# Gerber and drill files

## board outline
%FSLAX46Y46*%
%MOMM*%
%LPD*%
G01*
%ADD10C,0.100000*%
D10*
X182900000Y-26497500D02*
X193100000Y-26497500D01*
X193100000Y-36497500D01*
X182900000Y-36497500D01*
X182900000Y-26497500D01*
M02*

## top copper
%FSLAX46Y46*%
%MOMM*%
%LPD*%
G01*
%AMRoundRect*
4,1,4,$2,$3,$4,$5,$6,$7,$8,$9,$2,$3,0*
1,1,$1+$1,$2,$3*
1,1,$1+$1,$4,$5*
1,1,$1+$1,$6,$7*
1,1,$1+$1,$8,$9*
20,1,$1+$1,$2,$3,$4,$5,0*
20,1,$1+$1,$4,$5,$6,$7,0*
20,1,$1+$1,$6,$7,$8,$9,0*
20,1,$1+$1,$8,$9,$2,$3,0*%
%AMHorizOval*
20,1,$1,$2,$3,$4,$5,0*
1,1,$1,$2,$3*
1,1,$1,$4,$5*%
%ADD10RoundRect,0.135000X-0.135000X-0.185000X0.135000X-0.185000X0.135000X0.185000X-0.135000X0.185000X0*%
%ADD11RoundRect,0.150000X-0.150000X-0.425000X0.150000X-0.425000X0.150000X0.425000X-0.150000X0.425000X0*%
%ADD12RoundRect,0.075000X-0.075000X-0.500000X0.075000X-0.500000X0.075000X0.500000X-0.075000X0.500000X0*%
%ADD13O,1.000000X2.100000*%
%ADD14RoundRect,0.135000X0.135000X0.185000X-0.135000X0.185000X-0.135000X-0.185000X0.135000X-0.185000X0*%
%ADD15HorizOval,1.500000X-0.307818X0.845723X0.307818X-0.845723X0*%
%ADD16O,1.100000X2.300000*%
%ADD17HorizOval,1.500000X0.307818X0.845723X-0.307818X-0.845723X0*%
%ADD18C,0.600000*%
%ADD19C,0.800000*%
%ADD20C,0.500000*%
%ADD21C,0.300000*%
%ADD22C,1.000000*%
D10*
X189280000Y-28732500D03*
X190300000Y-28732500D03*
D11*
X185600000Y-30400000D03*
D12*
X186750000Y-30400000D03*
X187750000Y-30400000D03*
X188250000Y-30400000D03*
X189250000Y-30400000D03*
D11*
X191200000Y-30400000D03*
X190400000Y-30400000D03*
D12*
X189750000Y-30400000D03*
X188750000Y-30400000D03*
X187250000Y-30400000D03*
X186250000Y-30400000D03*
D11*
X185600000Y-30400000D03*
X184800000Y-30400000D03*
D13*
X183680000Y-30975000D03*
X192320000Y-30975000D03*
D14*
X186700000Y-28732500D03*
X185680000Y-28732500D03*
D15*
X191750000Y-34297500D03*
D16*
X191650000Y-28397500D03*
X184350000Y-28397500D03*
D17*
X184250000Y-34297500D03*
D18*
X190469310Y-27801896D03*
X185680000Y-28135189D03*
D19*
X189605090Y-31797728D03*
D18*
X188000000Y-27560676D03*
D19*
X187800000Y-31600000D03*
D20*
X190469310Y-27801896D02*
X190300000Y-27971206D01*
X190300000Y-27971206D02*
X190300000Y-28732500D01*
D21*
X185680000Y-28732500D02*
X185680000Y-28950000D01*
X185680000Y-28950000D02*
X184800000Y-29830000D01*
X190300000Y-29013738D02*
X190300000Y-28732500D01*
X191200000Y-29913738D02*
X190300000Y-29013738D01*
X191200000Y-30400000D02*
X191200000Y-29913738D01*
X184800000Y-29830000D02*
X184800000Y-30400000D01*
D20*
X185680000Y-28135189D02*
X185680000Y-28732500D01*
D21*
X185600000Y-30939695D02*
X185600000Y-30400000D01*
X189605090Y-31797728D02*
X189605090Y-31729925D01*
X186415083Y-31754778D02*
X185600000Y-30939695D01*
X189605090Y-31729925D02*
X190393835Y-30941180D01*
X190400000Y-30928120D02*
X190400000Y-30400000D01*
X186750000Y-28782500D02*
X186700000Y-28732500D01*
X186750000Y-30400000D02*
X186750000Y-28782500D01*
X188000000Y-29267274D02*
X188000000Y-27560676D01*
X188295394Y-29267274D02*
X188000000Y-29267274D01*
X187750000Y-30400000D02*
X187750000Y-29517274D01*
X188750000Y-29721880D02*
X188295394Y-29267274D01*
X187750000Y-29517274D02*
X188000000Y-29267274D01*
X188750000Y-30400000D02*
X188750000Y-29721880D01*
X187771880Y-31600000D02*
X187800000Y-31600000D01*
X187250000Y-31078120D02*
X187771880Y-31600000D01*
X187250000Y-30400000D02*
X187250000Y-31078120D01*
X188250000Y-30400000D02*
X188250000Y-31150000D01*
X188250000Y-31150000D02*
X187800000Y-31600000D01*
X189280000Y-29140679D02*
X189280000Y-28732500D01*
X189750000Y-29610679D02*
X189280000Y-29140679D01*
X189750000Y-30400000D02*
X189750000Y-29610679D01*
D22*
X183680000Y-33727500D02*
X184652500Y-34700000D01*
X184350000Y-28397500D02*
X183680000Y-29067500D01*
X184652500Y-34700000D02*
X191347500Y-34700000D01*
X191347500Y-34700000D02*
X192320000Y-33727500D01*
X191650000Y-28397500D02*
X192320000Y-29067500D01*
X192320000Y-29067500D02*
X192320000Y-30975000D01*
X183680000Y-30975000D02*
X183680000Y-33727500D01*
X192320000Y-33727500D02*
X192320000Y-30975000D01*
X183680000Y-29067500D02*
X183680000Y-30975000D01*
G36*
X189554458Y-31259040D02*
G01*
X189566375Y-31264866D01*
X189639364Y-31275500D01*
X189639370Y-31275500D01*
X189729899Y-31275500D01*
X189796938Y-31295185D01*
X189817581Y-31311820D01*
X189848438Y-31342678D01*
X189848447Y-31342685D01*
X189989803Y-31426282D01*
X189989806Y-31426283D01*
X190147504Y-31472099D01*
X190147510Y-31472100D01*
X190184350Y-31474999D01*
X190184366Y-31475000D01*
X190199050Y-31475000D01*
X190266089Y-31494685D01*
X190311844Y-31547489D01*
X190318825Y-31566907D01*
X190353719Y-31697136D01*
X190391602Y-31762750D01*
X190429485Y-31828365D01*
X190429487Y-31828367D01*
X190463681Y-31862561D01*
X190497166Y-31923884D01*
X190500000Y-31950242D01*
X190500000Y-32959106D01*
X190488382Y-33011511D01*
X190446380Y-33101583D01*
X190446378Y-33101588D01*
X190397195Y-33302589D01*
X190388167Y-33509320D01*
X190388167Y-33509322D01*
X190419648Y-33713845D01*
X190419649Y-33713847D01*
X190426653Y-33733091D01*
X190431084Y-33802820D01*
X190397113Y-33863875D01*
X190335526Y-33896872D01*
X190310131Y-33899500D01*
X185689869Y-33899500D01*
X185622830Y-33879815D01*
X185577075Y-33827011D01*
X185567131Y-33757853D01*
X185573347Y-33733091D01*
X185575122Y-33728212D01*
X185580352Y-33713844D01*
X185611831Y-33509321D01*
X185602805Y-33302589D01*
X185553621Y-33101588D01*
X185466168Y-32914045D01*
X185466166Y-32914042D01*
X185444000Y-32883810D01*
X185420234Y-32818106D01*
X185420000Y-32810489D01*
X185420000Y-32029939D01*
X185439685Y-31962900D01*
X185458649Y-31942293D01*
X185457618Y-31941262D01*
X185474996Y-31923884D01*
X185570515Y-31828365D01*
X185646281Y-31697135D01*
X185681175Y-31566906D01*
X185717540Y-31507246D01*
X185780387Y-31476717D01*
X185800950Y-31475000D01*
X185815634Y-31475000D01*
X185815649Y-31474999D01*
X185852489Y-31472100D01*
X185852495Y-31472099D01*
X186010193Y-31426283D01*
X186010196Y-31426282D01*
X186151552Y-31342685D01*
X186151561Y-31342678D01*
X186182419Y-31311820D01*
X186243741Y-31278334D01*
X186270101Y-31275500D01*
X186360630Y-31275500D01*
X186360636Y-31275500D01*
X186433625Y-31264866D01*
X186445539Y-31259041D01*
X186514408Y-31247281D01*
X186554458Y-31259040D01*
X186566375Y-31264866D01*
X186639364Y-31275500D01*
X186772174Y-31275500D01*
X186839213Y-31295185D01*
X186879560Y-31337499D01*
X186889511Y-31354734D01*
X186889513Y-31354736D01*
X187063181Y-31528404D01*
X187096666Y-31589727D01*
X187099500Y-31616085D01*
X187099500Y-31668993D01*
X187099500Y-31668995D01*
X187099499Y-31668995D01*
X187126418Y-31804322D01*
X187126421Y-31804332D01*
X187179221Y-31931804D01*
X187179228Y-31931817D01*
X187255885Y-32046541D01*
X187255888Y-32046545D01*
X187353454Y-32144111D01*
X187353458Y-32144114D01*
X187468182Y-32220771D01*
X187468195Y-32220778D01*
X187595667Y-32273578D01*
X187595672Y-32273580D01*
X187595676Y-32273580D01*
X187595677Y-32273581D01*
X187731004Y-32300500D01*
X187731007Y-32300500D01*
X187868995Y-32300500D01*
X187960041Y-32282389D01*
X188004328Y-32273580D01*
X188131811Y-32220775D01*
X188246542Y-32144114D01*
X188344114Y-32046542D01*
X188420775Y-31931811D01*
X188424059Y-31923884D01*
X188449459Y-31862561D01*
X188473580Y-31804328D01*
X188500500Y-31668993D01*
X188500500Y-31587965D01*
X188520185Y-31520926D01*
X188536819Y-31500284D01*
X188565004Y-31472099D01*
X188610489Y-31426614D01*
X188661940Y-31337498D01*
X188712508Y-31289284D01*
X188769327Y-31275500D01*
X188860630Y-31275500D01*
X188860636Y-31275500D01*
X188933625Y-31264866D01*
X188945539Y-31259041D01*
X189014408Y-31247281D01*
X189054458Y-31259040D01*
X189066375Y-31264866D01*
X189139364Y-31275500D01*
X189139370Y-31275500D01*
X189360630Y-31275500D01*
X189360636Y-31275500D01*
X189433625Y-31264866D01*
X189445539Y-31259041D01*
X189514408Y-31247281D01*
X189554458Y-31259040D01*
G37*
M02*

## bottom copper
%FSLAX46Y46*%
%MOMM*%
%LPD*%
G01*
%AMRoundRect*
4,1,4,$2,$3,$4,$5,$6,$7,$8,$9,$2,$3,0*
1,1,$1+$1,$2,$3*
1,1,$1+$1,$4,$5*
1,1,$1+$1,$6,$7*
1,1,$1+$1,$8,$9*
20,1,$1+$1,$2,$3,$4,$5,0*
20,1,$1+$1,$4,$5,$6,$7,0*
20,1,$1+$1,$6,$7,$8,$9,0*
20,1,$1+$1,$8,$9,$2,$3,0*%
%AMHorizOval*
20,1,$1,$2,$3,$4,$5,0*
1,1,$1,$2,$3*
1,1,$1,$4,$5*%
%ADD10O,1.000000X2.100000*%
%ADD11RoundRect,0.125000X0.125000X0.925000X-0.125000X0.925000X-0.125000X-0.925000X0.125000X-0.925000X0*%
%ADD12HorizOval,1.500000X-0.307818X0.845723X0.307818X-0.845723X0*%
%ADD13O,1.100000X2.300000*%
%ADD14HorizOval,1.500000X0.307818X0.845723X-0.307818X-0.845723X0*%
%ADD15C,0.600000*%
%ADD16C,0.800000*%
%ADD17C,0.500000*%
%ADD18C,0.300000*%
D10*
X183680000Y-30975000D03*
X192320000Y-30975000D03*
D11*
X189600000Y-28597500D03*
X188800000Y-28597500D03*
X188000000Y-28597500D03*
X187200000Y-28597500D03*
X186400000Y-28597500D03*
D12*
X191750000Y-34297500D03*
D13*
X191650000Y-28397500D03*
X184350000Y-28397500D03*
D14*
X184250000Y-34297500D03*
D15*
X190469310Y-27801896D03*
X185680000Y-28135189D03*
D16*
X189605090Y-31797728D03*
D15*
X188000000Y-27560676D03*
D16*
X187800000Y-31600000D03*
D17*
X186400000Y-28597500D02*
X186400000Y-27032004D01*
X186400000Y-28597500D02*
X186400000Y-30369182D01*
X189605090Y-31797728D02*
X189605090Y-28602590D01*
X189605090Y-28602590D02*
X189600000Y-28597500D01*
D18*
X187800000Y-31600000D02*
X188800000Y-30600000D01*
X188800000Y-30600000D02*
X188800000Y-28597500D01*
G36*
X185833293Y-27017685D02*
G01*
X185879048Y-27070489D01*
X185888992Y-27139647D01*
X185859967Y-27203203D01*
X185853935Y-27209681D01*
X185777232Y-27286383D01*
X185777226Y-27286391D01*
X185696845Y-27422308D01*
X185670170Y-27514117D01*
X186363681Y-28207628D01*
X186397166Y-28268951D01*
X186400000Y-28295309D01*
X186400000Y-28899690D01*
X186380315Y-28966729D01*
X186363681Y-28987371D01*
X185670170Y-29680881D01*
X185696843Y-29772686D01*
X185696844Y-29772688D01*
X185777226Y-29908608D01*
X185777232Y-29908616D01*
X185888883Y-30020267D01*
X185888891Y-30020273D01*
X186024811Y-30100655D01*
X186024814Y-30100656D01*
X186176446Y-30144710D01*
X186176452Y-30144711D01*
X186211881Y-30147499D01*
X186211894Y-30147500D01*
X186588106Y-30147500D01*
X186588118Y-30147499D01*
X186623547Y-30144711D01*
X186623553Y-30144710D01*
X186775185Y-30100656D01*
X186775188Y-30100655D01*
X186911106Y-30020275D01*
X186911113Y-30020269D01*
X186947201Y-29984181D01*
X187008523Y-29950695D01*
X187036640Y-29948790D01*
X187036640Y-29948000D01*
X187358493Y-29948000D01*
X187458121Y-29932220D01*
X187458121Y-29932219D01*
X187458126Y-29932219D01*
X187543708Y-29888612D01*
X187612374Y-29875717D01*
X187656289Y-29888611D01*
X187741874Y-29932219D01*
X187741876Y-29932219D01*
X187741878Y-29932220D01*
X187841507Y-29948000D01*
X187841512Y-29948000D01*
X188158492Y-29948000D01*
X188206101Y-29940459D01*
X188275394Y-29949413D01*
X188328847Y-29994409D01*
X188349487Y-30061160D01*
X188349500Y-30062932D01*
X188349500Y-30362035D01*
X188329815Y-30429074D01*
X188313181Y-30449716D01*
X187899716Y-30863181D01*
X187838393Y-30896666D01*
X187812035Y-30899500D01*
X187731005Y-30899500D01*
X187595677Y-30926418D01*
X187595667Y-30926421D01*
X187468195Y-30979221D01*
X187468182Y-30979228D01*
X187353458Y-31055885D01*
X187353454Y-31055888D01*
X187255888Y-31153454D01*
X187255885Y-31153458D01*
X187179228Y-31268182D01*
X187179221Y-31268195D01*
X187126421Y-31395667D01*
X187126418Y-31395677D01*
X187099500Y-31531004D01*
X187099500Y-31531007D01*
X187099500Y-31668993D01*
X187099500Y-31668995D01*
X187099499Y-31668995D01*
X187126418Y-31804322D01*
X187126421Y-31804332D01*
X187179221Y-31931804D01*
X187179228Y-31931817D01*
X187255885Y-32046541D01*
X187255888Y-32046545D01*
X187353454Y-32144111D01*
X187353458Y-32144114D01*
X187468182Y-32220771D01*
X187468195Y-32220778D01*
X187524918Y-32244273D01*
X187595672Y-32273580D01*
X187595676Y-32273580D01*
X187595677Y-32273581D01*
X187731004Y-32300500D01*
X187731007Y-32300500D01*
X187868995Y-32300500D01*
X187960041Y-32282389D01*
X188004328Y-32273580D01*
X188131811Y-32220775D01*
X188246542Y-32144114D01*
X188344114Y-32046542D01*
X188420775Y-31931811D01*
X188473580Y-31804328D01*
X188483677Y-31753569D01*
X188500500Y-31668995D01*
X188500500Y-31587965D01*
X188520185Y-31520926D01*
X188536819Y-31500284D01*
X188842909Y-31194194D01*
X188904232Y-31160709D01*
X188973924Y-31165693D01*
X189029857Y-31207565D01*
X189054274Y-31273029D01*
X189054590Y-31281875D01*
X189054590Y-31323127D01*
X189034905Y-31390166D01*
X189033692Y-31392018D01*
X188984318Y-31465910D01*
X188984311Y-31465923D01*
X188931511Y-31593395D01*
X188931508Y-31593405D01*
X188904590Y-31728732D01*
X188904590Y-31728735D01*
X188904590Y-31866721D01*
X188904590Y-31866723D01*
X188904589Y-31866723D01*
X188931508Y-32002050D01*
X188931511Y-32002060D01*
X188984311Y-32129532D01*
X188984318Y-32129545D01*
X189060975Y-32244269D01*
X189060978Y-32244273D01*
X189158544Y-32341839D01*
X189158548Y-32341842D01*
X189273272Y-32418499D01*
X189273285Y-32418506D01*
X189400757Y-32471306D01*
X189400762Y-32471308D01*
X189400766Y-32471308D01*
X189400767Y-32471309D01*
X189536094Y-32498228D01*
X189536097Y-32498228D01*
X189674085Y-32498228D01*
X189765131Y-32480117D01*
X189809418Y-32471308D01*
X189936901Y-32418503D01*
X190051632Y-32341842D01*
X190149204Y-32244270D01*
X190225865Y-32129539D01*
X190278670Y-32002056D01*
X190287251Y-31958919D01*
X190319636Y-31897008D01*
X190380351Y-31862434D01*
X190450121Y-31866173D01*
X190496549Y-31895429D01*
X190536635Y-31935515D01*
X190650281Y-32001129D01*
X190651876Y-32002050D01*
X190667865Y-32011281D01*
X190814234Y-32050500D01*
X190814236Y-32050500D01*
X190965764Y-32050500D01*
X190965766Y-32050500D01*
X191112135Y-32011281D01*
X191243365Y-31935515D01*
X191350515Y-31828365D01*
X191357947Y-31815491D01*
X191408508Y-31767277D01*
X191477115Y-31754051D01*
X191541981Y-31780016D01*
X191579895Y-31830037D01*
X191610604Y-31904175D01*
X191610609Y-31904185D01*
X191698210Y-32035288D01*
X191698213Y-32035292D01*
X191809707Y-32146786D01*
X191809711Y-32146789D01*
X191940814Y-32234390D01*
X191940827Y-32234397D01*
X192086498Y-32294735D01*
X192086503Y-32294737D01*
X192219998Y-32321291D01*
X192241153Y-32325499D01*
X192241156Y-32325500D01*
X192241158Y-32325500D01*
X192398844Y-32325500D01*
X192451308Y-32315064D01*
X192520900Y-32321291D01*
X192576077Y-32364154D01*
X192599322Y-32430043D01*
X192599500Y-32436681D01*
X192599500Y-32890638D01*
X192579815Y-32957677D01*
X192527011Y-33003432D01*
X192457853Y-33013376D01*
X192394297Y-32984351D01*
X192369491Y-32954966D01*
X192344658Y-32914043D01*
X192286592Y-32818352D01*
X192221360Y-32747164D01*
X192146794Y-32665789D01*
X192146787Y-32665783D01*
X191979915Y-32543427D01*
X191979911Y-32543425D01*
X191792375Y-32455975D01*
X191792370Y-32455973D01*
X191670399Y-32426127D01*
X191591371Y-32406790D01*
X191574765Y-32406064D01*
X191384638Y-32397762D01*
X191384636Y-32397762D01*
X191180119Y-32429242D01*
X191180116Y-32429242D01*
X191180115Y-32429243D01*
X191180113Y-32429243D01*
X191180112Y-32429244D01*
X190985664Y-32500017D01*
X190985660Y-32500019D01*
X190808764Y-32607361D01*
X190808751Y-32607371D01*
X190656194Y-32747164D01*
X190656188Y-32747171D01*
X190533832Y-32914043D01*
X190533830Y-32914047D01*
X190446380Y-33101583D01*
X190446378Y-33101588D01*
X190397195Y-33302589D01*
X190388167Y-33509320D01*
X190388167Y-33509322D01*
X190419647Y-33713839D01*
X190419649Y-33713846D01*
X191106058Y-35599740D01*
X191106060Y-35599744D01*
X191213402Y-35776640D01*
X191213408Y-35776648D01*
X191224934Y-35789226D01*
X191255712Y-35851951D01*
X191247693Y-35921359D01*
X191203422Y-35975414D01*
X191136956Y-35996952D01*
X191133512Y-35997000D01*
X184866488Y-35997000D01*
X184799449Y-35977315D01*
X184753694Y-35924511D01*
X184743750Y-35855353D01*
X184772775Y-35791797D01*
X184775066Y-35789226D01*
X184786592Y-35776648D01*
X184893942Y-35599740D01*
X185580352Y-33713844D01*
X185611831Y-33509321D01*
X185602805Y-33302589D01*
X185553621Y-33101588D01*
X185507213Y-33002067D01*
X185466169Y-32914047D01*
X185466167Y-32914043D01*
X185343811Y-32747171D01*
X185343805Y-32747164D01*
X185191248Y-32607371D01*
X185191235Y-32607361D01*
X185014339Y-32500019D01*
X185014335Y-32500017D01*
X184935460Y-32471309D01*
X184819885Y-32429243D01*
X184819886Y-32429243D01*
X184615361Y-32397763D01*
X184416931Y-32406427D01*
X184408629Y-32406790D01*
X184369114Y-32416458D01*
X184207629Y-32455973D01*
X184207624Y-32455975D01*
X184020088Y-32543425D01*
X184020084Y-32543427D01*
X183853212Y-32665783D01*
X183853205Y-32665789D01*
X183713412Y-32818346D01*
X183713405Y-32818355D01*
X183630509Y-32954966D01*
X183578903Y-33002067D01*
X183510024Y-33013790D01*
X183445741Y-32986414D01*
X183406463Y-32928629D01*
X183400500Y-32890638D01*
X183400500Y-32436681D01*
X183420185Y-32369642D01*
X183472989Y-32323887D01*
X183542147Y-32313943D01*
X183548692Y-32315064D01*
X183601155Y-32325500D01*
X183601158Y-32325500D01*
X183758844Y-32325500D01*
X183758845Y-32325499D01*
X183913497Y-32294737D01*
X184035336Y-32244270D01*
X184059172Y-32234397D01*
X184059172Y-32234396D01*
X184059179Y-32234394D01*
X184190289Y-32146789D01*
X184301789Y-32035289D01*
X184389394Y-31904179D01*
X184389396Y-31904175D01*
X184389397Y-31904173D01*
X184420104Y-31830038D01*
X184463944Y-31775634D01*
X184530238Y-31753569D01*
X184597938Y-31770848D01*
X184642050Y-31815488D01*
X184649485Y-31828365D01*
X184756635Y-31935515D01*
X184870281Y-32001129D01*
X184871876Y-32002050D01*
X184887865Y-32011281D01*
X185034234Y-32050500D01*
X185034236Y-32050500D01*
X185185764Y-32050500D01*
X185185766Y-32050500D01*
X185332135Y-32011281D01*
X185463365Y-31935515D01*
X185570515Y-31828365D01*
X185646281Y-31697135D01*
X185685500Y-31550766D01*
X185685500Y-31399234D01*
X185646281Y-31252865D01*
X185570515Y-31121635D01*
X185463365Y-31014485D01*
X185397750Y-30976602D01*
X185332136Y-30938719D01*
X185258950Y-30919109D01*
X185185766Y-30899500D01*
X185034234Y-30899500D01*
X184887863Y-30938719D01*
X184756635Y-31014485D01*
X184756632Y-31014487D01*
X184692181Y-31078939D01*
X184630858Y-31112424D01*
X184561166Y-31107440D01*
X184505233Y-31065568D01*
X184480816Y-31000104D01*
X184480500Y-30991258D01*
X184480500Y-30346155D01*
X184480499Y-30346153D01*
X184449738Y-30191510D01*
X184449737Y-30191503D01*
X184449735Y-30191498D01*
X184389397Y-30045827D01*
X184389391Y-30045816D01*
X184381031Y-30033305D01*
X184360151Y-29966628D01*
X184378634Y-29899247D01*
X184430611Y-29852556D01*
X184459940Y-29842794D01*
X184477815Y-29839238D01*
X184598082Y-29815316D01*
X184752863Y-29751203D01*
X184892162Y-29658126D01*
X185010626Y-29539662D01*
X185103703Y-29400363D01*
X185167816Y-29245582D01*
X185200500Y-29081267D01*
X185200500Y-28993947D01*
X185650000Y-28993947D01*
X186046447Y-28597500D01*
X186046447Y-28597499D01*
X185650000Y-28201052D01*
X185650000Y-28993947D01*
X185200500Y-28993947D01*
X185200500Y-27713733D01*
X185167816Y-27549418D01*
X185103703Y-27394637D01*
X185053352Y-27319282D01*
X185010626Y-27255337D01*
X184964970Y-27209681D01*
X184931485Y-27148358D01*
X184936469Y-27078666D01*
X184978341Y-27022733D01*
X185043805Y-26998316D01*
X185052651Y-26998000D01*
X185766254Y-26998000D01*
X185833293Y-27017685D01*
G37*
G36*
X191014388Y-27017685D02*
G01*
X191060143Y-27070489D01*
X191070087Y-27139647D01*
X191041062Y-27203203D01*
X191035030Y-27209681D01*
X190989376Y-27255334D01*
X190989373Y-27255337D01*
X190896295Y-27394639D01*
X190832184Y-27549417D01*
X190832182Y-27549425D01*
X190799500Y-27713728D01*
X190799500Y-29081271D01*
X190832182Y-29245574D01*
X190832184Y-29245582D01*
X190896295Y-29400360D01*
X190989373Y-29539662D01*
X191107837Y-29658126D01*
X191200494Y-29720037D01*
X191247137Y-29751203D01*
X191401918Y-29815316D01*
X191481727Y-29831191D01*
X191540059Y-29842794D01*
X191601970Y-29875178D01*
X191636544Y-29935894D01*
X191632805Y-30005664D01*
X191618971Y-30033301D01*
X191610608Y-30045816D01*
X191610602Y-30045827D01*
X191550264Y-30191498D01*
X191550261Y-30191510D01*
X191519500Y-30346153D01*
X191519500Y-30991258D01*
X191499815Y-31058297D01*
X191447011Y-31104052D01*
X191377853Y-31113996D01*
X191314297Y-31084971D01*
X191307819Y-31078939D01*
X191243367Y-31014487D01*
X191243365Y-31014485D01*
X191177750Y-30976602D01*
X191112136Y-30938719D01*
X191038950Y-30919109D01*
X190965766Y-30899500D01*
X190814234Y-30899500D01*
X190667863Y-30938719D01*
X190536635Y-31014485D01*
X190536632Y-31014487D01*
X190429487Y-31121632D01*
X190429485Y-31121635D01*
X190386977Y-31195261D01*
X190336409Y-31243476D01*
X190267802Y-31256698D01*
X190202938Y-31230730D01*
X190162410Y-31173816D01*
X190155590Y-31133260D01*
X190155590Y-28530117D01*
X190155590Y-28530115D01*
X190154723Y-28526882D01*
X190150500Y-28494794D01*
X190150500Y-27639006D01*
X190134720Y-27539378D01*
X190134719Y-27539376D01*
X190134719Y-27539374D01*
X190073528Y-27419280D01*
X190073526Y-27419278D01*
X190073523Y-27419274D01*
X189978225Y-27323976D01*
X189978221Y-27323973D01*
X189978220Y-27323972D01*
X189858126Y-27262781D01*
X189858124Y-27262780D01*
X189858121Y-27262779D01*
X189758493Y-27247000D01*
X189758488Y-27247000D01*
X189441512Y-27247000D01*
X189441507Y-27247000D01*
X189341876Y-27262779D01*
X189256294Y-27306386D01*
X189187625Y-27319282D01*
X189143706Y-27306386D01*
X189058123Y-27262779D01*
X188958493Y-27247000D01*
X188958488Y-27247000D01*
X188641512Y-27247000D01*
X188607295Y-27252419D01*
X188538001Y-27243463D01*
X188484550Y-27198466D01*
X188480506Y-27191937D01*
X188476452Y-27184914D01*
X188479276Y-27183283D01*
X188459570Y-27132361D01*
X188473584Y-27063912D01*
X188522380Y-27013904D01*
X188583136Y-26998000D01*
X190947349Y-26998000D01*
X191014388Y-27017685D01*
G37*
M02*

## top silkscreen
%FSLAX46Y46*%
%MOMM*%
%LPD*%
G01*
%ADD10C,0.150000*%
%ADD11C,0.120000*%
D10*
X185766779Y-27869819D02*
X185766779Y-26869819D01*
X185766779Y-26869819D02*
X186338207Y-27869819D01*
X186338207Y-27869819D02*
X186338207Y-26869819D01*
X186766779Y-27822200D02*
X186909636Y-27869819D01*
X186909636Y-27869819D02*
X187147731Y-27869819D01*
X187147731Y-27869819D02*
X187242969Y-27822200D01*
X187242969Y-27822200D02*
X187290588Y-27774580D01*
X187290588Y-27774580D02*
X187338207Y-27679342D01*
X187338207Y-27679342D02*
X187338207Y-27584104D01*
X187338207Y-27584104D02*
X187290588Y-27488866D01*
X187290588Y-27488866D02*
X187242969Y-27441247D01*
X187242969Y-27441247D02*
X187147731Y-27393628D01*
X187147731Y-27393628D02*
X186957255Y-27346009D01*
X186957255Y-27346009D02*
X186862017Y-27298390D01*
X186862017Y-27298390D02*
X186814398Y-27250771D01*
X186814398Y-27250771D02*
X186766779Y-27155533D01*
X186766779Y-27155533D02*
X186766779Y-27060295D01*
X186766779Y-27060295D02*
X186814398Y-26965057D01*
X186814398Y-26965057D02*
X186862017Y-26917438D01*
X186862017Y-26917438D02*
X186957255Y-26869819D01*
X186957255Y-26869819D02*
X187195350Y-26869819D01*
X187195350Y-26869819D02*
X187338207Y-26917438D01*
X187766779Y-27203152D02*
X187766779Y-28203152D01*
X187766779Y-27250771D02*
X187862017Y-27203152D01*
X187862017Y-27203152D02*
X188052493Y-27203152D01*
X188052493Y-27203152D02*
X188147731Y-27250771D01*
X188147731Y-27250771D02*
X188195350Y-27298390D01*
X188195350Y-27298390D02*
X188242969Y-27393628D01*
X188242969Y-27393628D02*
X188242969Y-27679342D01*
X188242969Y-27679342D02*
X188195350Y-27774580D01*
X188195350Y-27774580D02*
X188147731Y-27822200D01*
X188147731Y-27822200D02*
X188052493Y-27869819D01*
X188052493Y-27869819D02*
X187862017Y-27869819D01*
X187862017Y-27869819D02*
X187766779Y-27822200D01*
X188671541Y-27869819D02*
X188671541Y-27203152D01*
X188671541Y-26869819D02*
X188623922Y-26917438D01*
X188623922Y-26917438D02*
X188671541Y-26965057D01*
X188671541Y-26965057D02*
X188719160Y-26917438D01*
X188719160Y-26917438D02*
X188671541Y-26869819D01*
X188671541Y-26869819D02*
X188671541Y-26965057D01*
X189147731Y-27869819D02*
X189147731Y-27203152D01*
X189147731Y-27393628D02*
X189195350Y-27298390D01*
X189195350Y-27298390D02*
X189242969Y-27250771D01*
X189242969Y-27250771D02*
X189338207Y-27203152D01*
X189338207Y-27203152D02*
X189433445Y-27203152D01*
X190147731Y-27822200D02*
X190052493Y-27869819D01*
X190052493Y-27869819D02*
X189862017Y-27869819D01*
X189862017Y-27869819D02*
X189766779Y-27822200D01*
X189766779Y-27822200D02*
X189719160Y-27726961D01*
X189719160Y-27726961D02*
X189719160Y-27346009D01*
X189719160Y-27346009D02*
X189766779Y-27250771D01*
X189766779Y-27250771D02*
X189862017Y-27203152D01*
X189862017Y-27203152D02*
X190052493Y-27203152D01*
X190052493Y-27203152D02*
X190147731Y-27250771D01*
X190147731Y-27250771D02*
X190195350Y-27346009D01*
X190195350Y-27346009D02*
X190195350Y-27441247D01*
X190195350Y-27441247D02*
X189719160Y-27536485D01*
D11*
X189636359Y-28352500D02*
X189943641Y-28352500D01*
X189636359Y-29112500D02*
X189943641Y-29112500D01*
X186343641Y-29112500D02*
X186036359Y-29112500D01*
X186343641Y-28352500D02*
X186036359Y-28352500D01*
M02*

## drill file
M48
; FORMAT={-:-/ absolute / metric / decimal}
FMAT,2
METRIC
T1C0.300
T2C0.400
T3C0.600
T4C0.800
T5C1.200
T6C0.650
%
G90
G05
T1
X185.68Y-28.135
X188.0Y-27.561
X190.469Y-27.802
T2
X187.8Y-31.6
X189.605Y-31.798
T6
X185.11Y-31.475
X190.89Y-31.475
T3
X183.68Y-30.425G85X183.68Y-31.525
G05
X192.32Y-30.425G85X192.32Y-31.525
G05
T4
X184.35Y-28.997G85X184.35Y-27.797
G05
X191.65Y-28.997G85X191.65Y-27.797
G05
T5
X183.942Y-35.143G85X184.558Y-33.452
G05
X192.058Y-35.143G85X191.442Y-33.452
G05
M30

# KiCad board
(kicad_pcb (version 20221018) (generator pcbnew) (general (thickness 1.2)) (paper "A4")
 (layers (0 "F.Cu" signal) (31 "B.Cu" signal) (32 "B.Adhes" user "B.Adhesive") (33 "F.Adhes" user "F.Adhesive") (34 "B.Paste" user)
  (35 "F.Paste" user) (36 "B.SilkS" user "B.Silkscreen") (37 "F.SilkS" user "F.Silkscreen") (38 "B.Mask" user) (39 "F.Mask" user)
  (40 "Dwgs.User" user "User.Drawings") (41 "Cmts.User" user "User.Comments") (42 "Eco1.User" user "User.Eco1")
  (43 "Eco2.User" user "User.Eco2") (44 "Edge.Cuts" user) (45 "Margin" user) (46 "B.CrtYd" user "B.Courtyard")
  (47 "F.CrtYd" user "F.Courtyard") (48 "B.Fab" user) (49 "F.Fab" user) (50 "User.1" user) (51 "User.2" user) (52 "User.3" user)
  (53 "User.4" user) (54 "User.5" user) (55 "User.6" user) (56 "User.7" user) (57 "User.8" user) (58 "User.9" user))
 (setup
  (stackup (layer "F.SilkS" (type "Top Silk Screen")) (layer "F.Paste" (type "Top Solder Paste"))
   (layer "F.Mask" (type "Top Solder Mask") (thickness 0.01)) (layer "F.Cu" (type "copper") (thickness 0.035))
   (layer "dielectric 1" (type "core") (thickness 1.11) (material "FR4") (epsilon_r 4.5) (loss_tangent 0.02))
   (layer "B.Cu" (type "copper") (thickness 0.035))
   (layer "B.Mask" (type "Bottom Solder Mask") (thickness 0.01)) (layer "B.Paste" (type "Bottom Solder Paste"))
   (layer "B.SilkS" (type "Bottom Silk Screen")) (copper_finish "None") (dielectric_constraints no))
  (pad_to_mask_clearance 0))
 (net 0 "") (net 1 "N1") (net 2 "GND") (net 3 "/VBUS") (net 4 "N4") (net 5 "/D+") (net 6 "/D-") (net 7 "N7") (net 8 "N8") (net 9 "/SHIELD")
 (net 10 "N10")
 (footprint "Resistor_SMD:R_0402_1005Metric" (layer "F.Cu") (at 189.79 28.7325)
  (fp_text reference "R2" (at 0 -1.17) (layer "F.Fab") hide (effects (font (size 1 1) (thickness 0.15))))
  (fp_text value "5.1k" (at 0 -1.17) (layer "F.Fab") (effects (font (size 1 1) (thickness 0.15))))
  (fp_line (start -0.153641 -0.38) (end 0.153641 -0.38) (stroke (width 0.12) (type solid)) (layer "F.SilkS"))
  (fp_line (start -0.153641 0.38) (end 0.153641 0.38) (stroke (width 0.12) (type solid)) (layer "F.SilkS"))
  (pad "1" smd roundrect (at -0.51 0) (size 0.54 0.64) (layers "F.Cu" "F.Paste" "F.Mask") (roundrect_rratio 0.25) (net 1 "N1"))
  (pad "2" smd roundrect (at 0.51 0) (size 0.54 0.64) (layers "F.Cu" "F.Paste" "F.Mask") (roundrect_rratio 0.25) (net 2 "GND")))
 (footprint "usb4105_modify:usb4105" (layer "F.Cu") (at 187.98 39.92)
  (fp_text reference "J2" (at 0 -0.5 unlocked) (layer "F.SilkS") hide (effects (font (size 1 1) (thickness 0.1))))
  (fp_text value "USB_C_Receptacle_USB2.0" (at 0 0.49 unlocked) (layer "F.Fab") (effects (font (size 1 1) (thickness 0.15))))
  (pad "" np_thru_hole circle (at -2.87 -8.445) (size 0.65 0.65) (drill 0.65) (layers "F&B.Cu" "*.Mask"))
  (pad "" np_thru_hole circle (at 2.91 -8.445) (size 0.65 0.65) (drill 0.65) (layers "F&B.Cu" "*.Mask"))
  (pad "A4" smd roundrect (at -2.38 -9.52) (size 0.6 1.15) (layers "F.Cu" "F.Paste" "F.Mask") (roundrect_rratio 0.25) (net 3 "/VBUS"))
  (pad "A5" smd roundrect (at -1.23 -9.52) (size 0.3 1.15) (layers "F.Cu" "F.Paste" "F.Mask") (roundrect_rratio 0.25) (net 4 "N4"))
  (pad "A6" smd roundrect (at -0.23 -9.52) (size 0.3 1.15) (layers "F.Cu" "F.Paste" "F.Mask") (roundrect_rratio 0.25) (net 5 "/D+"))
  (pad "A7" smd roundrect (at 0.27 -9.52) (size 0.3 1.15) (layers "F.Cu" "F.Paste" "F.Mask") (roundrect_rratio 0.25) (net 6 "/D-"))
  (pad "A8" smd roundrect (at 1.27 -9.52) (size 0.3 1.15) (layers "F.Cu" "F.Paste" "F.Mask") (roundrect_rratio 0.25) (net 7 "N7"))
  (pad "A12" smd roundrect (at 3.22 -9.52) (size 0.6 1.15) (layers "F.Cu" "F.Paste" "F.Mask") (roundrect_rratio 0.25) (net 2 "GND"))
  (pad "B4" smd roundrect (at 2.42 -9.52) (size 0.6 1.15) (layers "F.Cu" "F.Paste" "F.Mask") (roundrect_rratio 0.25) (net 3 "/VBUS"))
  (pad "B5" smd roundrect (at 1.77 -9.52) (size 0.3 1.15) (layers "F.Cu" "F.Paste" "F.Mask") (roundrect_rratio 0.25) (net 1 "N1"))
  (pad "B6" smd roundrect (at 0.77 -9.52) (size 0.3 1.15) (layers "F.Cu" "F.Paste" "F.Mask") (roundrect_rratio 0.25) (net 5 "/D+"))
  (pad "B7" smd roundrect (at -0.73 -9.52) (size 0.3 1.15) (layers "F.Cu" "F.Paste" "F.Mask") (roundrect_rratio 0.25) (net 6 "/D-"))
  (pad "B8" smd roundrect (at -1.73 -9.52) (size 0.3 1.15) (layers "F.Cu" "F.Paste" "F.Mask") (roundrect_rratio 0.25) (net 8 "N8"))
  (pad "B9" smd roundrect (at -2.38 -9.52) (size 0.6 1.15) (layers "F.Cu" "F.Paste" "F.Mask") (roundrect_rratio 0.25) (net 3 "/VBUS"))
  (pad "B12" smd roundrect (at -3.18 -9.52) (size 0.6 1.15) (layers "F.Cu" "F.Paste" "F.Mask") (roundrect_rratio 0.25) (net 2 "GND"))
  (pad "S1" thru_hole oval (at -4.3 -8.945) (size 1 2.1) (drill oval 0.6 1.7) (layers "*.Cu" "*.Mask" "F.Paste") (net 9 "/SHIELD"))
  (pad "S1" thru_hole oval (at 4.34 -8.945) (size 1 2.1) (drill oval 0.6 1.7) (layers "*.Cu" "*.Mask" "F.Paste") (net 9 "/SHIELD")))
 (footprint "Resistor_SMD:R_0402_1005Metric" (layer "F.Cu") (at 186.19 28.7325 180)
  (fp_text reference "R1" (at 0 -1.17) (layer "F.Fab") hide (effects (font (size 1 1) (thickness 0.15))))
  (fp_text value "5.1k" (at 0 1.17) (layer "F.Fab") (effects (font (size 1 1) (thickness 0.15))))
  (fp_line (start -0.153641 -0.38) (end 0.153641 -0.38) (stroke (width 0.12) (type solid)) (layer "F.SilkS"))
  (fp_line (start -0.153641 0.38) (end 0.153641 0.38) (stroke (width 0.12) (type solid)) (layer "F.SilkS"))
  (pad "1" smd roundrect (at -0.51 0 180) (size 0.54 0.64) (layers "F.Cu" "F.Paste" "F.Mask") (roundrect_rratio 0.25) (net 4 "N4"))
  (pad "2" smd roundrect (at 0.51 0 180) (size 0.54 0.64) (layers "F.Cu" "F.Paste" "F.Mask") (roundrect_rratio 0.25) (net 2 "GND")))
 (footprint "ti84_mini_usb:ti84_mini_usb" (layer "B.Cu") (at 188.25 38.1975 180)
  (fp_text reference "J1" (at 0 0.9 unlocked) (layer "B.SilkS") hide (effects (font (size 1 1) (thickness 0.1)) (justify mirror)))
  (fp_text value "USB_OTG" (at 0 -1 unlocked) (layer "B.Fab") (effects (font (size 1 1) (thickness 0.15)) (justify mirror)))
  (pad "1" smd roundrect (at -1.35 9.6 180) (size 0.5 2.1) (layers "B.Cu" "B.Paste" "B.Mask") (roundrect_rratio 0.25) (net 3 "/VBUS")
   (thermal_bridge_angle 45))
  (pad "2" smd roundrect (at -0.55 9.6 180) (size 0.5 2.1) (layers "B.Cu" "B.Paste" "B.Mask") (roundrect_rratio 0.25) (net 6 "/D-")
   (thermal_bridge_angle 45))
  (pad "3" smd roundrect (at 0.25 9.6 180) (size 0.5 2.1) (layers "B.Cu" "B.Paste" "B.Mask") (roundrect_rratio 0.25) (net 5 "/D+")
   (thermal_bridge_angle 45))
  (pad "4" smd roundrect (at 1.05 9.6 180) (size 0.5 2.1) (layers "B.Cu" "B.Paste" "B.Mask") (roundrect_rratio 0.25) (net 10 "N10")
   (thermal_bridge_angle 45))
  (pad "5" smd roundrect (at 1.85 9.6 180) (size 0.5 2.1) (layers "B.Cu" "B.Paste" "B.Mask") (roundrect_rratio 0.25) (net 2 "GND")
   (thermal_bridge_angle 45))
  (pad "6" thru_hole oval (at -3.5 3.9 200) (size 1.5 3.3) (drill oval 1.2 3) (layers "*.Cu" "*.Mask") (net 9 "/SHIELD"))
  (pad "6" thru_hole oval (at -3.4 9.8 180) (size 1.1 2.3) (drill oval 0.8 2) (layers "*.Cu" "*.Mask") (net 9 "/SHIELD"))
  (pad "6" thru_hole oval (at 3.9 9.8 180) (size 1.1 2.3) (drill oval 0.8 2) (layers "*.Cu" "*.Mask") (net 9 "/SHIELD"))
  (pad "6" thru_hole oval (at 4 3.9 160) (size 1.5 3.3) (drill oval 1.2 3) (layers "*.Cu" "*.Mask") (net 9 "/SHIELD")))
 (gr_rect (start 182.9 26.4975) (end 193.1 36.4975) (stroke (width 0.1) (type default)) (fill none) (layer "Edge.Cuts"))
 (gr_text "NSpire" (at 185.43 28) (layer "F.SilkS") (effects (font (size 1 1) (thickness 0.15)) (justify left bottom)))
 (segment (start 190.46931 27.801896) (end 190.3 27.971206) (width 0.5) (layer "F.Cu") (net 2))
 (segment (start 190.3 27.971206) (end 190.3 28.7325) (width 0.5) (layer "F.Cu") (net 2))
 (segment (start 185.68 28.7325) (end 185.68 28.95) (width 0.3) (layer "F.Cu") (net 2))
 (segment (start 185.68 28.95) (end 184.8 29.83) (width 0.3) (layer "F.Cu") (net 2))
 (segment (start 190.3 29.013738) (end 190.3 28.7325) (width 0.3) (layer "F.Cu") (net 2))
 (segment (start 191.2 29.913738) (end 190.3 29.013738) (width 0.3) (layer "F.Cu") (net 2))
 (segment (start 191.2 30.4) (end 191.2 29.913738) (width 0.3) (layer "F.Cu") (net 2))
 (segment (start 184.8 29.83) (end 184.8 30.4) (width 0.3) (layer "F.Cu") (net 2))
 (segment (start 185.68 28.135189) (end 185.68 28.7325) (width 0.5) (layer "F.Cu") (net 2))
 (via (at 190.46931 27.801896) (size 0.6) (drill 0.3) (layers "F.Cu" "B.Cu") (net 2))
 (via (at 185.68 28.135189) (size 0.6) (drill 0.3) (layers "F.Cu" "B.Cu") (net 2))
 (segment (start 186.4 28.5975) (end 186.4 27.032004) (width 0.5) (layer "B.Cu") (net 2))
 (segment (start 186.4 28.5975) (end 186.4 30.369182) (width 0.5) (layer "B.Cu") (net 2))
 (segment (start 185.6 30.939695) (end 185.6 30.4) (width 0.3) (layer "F.Cu") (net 3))
 (segment (start 189.60509 31.797728) (end 189.60509 31.729925) (width 0.3) (layer "F.Cu") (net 3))
 (segment (start 186.415083 31.754778) (end 185.6 30.939695) (width 0.3) (layer "F.Cu") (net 3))
 (segment (start 189.60509 31.729925) (end 190.393835 30.94118) (width 0.3) (layer "F.Cu") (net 3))
 (segment (start 190.4 30.92812) (end 190.4 30.4) (width 0.3) (layer "F.Cu") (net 3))
 (via (at 189.60509 31.797728) (size 0.8) (drill 0.4) (layers "F.Cu" "B.Cu") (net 3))
 (segment (start 189.60509 31.797728) (end 189.60509 28.60259) (width 0.5) (layer "B.Cu") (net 3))
 (segment (start 189.60509 28.60259) (end 189.6 28.5975) (width 0.5) (layer "B.Cu") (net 3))
 (segment (start 186.75 28.7825) (end 186.7 28.7325) (width 0.3) (layer "F.Cu") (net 4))
 (segment (start 186.75 30.4) (end 186.75 28.7825) (width 0.3) (layer "F.Cu") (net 4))
 (segment (start 188 29.267274) (end 188 27.560676) (width 0.3) (layer "F.Cu") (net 5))
 (segment (start 188.295394 29.267274) (end 188 29.267274) (width 0.3) (layer "F.Cu") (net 5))
 (segment (start 187.75 30.4) (end 187.75 29.517274) (width 0.3) (layer "F.Cu") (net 5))
 (segment (start 188.75 29.72188) (end 188.295394 29.267274) (width 0.3) (layer "F.Cu") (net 5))
 (segment (start 187.75 29.517274) (end 188 29.267274) (width 0.3) (layer "F.Cu") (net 5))
 (segment (start 188.75 30.4) (end 188.75 29.72188) (width 0.3) (layer "F.Cu") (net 5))
 (via (at 188 27.560676) (size 0.6) (drill 0.3) (layers "F.Cu" "B.Cu") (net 5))
 (segment (start 187.77188 31.6) (end 187.8 31.6) (width 0.3) (layer "F.Cu") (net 6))
 (segment (start 187.25 31.07812) (end 187.77188 31.6) (width 0.3) (layer "F.Cu") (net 6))
 (segment (start 187.25 30.4) (end 187.25 31.07812) (width 0.3) (layer "F.Cu") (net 6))
 (segment (start 188.25 30.4) (end 188.25 31.15) (width 0.3) (layer "F.Cu") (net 6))
 (segment (start 188.25 31.15) (end 187.8 31.6) (width 0.3) (layer "F.Cu") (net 6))
 (via (at 187.8 31.6) (size 0.8) (drill 0.4) (layers "F.Cu" "B.Cu") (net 6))
 (segment (start 187.8 31.6) (end 188.8 30.6) (width 0.3) (layer "B.Cu") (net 6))
 (segment (start 188.8 30.6) (end 188.8 28.5975) (width 0.3) (layer "B.Cu") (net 6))
 (segment (start 189.28 29.140679) (end 189.28 28.7325) (width 0.3) (layer "F.Cu") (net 1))
 (segment (start 189.75 29.610679) (end 189.28 29.140679) (width 0.3) (layer "F.Cu") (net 1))
 (segment (start 189.75 30.4) (end 189.75 29.610679) (width 0.3) (layer "F.Cu") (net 1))
 (segment (start 183.68 33.7275) (end 184.6525 34.7) (width 1) (layer "F.Cu") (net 9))
 (segment (start 184.35 28.3975) (end 183.68 29.0675) (width 1) (layer "F.Cu") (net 9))
 (segment (start 184.6525 34.7) (end 191.3475 34.7) (width 1) (layer "F.Cu") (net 9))
 (segment (start 191.3475 34.7) (end 192.32 33.7275) (width 1) (layer "F.Cu") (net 9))
 (segment (start 191.65 28.3975) (end 192.32 29.0675) (width 1) (layer "F.Cu") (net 9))
 (segment (start 192.32 29.0675) (end 192.32 30.975) (width 1) (layer "F.Cu") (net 9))
 (segment (start 183.68 30.975) (end 183.68 33.7275) (width 1) (layer "F.Cu") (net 9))
 (segment (start 192.32 33.7275) (end 192.32 30.975) (width 1) (layer "F.Cu") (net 9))
 (segment (start 183.68 29.0675) (end 183.68 30.975) (width 1) (layer "F.Cu") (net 9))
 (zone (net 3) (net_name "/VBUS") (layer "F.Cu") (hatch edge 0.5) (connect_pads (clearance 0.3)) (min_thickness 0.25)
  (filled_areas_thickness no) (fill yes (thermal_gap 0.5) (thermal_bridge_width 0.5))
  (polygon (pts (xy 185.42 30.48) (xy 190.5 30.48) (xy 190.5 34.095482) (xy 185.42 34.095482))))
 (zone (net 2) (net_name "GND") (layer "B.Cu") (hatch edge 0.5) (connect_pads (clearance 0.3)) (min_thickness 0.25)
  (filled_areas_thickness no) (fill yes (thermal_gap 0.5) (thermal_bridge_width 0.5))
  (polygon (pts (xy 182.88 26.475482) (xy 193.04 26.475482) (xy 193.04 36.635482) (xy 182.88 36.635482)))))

